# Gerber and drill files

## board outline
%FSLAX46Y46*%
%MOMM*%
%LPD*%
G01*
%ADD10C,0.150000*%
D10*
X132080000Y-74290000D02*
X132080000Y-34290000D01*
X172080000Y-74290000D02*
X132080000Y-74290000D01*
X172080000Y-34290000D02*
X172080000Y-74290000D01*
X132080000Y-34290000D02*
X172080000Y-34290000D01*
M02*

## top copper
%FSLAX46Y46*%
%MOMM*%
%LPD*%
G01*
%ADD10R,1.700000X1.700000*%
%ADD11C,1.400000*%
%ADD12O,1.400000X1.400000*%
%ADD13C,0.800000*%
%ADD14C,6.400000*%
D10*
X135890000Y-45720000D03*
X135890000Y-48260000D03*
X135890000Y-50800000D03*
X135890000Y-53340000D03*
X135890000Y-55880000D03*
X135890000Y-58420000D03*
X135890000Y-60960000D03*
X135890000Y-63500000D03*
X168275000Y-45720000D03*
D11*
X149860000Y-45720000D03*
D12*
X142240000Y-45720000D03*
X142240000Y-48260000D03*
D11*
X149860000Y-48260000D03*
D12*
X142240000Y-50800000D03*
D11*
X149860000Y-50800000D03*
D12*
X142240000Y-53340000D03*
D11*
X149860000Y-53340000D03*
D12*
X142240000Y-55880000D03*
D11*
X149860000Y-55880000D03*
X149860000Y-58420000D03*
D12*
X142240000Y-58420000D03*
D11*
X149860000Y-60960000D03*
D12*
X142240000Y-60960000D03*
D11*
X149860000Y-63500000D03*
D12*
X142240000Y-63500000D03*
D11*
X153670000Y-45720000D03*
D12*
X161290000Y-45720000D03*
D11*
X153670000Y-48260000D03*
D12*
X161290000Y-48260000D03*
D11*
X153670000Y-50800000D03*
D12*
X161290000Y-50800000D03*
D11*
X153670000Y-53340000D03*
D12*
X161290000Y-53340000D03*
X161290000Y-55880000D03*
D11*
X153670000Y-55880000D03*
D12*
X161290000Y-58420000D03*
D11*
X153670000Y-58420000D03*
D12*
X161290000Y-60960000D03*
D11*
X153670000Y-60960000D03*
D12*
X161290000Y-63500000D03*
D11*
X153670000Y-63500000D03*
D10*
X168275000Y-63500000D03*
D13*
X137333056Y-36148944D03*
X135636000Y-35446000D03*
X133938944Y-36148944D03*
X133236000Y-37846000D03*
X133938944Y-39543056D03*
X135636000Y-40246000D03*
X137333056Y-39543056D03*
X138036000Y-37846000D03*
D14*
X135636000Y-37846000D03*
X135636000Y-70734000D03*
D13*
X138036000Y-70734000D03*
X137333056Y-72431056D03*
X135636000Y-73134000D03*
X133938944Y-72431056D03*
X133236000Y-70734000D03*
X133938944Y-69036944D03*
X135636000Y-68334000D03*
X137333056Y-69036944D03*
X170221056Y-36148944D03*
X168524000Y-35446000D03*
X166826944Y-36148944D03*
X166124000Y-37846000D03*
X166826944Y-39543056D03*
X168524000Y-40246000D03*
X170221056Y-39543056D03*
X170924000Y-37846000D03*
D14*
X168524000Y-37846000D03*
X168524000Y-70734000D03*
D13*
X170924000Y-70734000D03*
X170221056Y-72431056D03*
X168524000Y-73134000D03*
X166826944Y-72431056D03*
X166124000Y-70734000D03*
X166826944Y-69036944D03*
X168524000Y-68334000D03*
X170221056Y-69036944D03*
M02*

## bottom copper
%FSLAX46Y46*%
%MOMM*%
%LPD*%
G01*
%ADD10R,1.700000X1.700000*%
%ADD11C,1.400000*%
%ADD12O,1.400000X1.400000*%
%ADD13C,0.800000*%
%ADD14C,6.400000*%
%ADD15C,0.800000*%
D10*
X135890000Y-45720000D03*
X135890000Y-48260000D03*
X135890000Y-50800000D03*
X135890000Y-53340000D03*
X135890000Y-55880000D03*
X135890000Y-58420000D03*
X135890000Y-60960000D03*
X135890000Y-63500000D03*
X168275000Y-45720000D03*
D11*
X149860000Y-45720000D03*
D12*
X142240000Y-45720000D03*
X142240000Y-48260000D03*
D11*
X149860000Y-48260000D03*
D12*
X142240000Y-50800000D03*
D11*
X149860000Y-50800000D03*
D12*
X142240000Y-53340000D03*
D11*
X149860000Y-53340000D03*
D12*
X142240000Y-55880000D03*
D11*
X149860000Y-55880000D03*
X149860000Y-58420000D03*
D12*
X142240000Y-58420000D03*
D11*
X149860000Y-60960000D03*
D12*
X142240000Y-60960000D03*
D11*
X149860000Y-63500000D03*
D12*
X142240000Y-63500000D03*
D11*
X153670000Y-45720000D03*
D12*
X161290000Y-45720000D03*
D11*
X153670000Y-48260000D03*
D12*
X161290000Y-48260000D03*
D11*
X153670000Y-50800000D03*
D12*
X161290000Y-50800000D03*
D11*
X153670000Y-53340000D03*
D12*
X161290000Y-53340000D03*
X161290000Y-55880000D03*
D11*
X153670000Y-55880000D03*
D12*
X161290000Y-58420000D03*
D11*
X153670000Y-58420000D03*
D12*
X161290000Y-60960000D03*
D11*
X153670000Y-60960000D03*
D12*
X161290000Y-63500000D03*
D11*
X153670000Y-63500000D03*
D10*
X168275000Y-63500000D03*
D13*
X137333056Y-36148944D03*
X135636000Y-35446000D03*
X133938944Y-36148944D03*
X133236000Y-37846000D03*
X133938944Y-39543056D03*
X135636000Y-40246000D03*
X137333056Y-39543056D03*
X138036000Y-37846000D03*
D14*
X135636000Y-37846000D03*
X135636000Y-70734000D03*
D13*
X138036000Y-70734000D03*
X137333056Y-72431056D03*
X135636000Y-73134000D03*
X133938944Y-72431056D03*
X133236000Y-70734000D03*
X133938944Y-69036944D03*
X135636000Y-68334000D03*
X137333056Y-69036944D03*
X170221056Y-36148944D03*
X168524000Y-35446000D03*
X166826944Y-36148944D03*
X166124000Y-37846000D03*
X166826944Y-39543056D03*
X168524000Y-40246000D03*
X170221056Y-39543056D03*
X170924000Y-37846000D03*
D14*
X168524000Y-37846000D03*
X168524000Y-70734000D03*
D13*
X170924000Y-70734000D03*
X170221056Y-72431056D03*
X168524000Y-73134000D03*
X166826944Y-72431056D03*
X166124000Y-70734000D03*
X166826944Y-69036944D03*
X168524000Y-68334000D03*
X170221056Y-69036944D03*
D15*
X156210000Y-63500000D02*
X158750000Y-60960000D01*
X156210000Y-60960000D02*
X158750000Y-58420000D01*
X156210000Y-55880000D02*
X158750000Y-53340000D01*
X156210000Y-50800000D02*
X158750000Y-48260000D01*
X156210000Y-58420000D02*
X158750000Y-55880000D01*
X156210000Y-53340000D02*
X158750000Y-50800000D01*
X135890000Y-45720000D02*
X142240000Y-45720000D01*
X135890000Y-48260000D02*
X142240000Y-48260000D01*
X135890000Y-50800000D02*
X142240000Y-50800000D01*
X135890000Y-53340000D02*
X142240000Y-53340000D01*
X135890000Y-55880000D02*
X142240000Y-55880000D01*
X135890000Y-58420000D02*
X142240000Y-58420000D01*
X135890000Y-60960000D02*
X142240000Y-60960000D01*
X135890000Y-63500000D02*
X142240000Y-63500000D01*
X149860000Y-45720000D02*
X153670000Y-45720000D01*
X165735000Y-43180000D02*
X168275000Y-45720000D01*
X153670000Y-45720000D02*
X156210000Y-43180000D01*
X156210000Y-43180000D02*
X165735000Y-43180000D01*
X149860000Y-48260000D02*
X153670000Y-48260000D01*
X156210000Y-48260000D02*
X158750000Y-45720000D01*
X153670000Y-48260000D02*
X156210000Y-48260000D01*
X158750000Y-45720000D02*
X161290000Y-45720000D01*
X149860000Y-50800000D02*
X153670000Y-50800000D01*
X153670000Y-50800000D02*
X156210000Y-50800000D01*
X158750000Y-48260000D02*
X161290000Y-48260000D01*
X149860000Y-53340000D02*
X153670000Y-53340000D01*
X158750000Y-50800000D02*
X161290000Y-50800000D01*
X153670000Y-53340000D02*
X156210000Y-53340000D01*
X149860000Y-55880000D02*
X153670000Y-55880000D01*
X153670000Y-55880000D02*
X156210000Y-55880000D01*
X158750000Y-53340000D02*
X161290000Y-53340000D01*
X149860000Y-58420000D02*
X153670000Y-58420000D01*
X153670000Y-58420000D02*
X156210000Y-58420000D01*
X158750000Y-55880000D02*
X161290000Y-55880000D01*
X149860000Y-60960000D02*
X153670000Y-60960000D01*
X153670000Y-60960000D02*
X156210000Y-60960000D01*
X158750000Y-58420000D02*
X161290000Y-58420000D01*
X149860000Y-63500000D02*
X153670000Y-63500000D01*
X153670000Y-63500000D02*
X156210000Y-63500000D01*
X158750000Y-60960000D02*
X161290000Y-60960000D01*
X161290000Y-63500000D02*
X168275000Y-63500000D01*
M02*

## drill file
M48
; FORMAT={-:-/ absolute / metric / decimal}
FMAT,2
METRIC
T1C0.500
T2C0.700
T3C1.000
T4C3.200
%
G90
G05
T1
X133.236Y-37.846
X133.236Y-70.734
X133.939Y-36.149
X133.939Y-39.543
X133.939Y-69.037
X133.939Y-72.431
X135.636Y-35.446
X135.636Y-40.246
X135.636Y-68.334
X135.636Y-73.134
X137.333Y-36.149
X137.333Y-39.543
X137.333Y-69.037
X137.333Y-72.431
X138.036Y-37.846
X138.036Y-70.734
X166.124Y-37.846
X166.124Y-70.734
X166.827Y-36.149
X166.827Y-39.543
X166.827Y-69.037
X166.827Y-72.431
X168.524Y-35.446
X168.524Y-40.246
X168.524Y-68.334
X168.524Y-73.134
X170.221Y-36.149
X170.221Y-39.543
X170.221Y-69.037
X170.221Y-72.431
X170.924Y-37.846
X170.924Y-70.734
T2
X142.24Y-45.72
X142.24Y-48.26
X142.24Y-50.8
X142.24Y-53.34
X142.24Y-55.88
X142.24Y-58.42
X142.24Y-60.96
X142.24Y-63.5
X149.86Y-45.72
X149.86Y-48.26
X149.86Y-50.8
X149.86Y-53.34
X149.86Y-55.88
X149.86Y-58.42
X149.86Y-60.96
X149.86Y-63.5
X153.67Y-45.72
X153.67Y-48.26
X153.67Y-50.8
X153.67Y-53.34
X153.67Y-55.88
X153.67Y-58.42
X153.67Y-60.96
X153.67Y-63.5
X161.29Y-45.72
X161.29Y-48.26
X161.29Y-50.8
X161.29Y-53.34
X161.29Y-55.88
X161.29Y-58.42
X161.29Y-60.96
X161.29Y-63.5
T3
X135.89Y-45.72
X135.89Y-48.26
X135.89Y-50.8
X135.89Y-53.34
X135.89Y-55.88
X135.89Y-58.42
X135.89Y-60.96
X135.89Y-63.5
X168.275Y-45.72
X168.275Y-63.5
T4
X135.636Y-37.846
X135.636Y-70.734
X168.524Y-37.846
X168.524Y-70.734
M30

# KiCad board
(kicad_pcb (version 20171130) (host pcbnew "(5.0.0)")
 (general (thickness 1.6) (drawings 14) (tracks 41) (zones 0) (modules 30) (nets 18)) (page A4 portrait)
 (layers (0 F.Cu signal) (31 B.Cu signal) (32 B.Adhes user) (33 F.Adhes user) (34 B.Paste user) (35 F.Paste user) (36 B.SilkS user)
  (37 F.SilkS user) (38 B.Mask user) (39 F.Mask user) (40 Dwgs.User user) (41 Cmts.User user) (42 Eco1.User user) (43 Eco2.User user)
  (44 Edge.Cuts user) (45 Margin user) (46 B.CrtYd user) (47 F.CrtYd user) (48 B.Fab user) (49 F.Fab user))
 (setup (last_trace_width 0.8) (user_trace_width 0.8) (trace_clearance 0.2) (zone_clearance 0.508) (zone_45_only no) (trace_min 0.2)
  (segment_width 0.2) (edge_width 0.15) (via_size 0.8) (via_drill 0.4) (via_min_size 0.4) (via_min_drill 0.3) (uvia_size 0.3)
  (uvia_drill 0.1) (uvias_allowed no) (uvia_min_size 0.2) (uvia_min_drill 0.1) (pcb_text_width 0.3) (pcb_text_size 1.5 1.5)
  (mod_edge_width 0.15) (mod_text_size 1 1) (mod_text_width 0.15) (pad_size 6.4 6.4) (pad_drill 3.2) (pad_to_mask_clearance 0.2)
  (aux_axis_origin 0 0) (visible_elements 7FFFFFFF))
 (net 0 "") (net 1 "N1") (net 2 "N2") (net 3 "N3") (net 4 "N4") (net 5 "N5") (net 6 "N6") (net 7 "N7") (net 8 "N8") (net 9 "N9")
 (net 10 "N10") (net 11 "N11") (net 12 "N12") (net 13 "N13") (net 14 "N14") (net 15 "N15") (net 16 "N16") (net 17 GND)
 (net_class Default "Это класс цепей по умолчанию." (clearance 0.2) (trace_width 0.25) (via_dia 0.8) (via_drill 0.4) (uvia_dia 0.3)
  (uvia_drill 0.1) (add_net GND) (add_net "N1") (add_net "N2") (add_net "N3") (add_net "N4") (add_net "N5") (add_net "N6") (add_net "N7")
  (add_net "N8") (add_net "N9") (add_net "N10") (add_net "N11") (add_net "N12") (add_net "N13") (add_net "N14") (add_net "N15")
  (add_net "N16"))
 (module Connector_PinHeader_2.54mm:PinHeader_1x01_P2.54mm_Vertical (layer F.Cu) (at 135.89 45.72)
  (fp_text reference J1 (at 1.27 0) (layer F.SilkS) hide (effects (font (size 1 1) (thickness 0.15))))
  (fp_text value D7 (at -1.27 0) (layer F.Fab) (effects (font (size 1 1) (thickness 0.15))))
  (pad 1 thru_hole rect (at 0 0) (size 1.7 1.7) (drill 1) (layers *.Cu *.Mask) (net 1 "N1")))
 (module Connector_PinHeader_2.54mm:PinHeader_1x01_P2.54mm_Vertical (layer F.Cu) (at 135.89 48.26)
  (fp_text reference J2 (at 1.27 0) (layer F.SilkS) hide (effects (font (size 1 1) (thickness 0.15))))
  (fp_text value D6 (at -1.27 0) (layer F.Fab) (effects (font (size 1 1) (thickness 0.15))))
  (pad 1 thru_hole rect (at 0 0) (size 1.7 1.7) (drill 1) (layers *.Cu *.Mask) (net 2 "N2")))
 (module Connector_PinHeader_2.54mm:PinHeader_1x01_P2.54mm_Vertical (layer F.Cu) (at 135.89 50.8)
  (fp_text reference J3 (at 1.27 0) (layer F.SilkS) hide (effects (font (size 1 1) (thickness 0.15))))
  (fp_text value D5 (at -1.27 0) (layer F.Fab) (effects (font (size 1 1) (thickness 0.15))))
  (pad 1 thru_hole rect (at 0 0) (size 1.7 1.7) (drill 1) (layers *.Cu *.Mask) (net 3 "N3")))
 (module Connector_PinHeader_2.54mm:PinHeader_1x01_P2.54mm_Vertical (layer F.Cu) (at 135.89 53.34)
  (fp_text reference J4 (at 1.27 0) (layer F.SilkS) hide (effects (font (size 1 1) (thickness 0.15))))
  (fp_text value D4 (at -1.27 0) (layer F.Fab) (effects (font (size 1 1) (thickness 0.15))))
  (pad 1 thru_hole rect (at 0 0) (size 1.7 1.7) (drill 1) (layers *.Cu *.Mask) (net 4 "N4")))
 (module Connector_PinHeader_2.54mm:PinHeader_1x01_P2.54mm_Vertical (layer F.Cu) (at 135.89 55.88)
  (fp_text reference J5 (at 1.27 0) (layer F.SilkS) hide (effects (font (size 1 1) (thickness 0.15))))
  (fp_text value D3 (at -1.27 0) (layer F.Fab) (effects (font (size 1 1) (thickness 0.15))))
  (pad 1 thru_hole rect (at 0 0) (size 1.7 1.7) (drill 1) (layers *.Cu *.Mask) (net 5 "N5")))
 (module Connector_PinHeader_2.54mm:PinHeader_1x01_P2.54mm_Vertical (layer F.Cu) (at 135.89 58.42)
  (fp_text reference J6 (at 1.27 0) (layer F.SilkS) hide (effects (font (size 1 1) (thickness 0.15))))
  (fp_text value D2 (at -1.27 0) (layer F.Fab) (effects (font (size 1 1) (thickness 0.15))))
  (pad 1 thru_hole rect (at 0 0) (size 1.7 1.7) (drill 1) (layers *.Cu *.Mask) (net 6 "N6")))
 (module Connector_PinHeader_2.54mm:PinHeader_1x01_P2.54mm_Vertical (layer F.Cu) (at 135.89 60.96)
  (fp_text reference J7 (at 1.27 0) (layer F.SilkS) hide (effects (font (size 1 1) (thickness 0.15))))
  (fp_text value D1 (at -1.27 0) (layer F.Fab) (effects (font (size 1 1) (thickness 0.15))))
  (pad 1 thru_hole rect (at 0 0) (size 1.7 1.7) (drill 1) (layers *.Cu *.Mask) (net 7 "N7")))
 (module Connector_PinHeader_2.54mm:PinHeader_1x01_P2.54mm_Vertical (layer F.Cu) (at 135.89 63.5)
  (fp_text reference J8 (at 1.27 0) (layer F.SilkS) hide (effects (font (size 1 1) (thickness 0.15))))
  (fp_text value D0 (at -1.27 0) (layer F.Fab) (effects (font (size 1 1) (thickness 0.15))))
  (pad 1 thru_hole rect (at 0 0) (size 1.7 1.7) (drill 1) (layers *.Cu *.Mask) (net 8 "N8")))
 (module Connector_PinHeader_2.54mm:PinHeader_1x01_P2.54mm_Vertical (layer F.Cu) (at 168.275 45.72)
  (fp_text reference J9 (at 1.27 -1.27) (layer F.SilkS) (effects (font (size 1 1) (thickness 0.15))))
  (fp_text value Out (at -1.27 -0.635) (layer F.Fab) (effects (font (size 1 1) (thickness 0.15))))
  (pad 1 thru_hole rect (at 0 0) (size 1.7 1.7) (drill 1) (layers *.Cu *.Mask) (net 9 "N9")))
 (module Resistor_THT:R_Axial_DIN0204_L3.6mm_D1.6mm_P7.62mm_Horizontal (layer F.Cu) (at 149.86 45.72 180)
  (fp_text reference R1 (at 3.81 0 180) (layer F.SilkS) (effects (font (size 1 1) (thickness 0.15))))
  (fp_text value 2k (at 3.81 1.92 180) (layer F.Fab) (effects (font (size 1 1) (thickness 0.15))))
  (pad 1 thru_hole circle (at 0 0 180) (size 1.4 1.4) (drill 0.7) (layers *.Cu *.Mask) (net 9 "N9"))
  (pad 2 thru_hole oval (at 7.62 0 180) (size 1.4 1.4) (drill 0.7) (layers *.Cu *.Mask) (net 1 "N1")))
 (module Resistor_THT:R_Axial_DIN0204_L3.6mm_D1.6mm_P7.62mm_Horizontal (layer F.Cu) (at 149.86 48.26 180)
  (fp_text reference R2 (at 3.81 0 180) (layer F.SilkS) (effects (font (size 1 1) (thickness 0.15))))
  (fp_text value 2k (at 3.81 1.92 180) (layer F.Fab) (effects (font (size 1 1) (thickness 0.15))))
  (pad 2 thru_hole oval (at 7.62 0 180) (size 1.4 1.4) (drill 0.7) (layers *.Cu *.Mask) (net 2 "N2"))
  (pad 1 thru_hole circle (at 0 0 180) (size 1.4 1.4) (drill 0.7) (layers *.Cu *.Mask) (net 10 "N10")))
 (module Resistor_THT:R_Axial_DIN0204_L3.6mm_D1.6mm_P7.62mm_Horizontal (layer F.Cu) (at 149.86 50.8 180)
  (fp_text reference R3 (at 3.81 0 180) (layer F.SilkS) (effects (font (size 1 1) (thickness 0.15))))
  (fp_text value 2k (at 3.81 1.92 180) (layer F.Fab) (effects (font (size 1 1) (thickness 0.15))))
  (pad 2 thru_hole oval (at 7.62 0 180) (size 1.4 1.4) (drill 0.7) (layers *.Cu *.Mask) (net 3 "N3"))
  (pad 1 thru_hole circle (at 0 0 180) (size 1.4 1.4) (drill 0.7) (layers *.Cu *.Mask) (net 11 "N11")))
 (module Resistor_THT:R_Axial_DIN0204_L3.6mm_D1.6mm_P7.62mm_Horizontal (layer F.Cu) (at 149.86 53.34 180)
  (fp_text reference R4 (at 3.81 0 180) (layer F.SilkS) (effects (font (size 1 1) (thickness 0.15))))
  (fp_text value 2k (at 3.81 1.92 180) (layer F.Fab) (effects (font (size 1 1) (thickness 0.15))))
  (pad 2 thru_hole oval (at 7.62 0 180) (size 1.4 1.4) (drill 0.7) (layers *.Cu *.Mask) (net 4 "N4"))
  (pad 1 thru_hole circle (at 0 0 180) (size 1.4 1.4) (drill 0.7) (layers *.Cu *.Mask) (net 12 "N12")))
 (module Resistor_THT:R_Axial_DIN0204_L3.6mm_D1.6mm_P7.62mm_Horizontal (layer F.Cu) (at 149.86 55.88 180)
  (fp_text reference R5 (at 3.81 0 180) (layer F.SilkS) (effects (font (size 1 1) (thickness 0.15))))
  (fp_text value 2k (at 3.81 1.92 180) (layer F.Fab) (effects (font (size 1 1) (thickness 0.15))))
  (pad 2 thru_hole oval (at 7.62 0 180) (size 1.4 1.4) (drill 0.7) (layers *.Cu *.Mask) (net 5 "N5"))
  (pad 1 thru_hole circle (at 0 0 180) (size 1.4 1.4) (drill 0.7) (layers *.Cu *.Mask) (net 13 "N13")))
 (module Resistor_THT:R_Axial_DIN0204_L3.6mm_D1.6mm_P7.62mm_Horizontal (layer F.Cu) (at 149.86 58.42 180)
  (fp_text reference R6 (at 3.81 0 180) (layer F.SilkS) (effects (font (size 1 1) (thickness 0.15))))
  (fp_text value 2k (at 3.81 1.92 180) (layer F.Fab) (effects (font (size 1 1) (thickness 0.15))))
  (pad 1 thru_hole circle (at 0 0 180) (size 1.4 1.4) (drill 0.7) (layers *.Cu *.Mask) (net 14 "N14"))
  (pad 2 thru_hole oval (at 7.62 0 180) (size 1.4 1.4) (drill 0.7) (layers *.Cu *.Mask) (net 6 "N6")))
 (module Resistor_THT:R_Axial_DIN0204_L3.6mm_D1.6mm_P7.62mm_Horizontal (layer F.Cu) (at 149.86 60.96 180)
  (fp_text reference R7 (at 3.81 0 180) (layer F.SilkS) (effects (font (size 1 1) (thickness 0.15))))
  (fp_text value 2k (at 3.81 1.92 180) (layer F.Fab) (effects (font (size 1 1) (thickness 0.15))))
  (pad 1 thru_hole circle (at 0 0 180) (size 1.4 1.4) (drill 0.7) (layers *.Cu *.Mask) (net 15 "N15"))
  (pad 2 thru_hole oval (at 7.62 0 180) (size 1.4 1.4) (drill 0.7) (layers *.Cu *.Mask) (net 7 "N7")))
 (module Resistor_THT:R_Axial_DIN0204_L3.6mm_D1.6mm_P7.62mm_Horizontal (layer F.Cu) (at 149.86 63.5 180)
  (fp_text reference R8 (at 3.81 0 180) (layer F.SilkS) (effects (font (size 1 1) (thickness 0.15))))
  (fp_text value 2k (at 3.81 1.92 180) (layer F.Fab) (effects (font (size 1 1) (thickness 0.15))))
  (pad 1 thru_hole circle (at 0 0 180) (size 1.4 1.4) (drill 0.7) (layers *.Cu *.Mask) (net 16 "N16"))
  (pad 2 thru_hole oval (at 7.62 0 180) (size 1.4 1.4) (drill 0.7) (layers *.Cu *.Mask) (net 8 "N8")))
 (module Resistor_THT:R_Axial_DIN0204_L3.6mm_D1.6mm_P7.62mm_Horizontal (layer F.Cu) (at 153.67 45.72)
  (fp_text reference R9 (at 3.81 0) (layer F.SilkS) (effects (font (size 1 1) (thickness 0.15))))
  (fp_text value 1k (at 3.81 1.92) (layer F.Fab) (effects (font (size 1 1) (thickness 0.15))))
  (pad 1 thru_hole circle (at 0 0) (size 1.4 1.4) (drill 0.7) (layers *.Cu *.Mask) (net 9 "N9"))
  (pad 2 thru_hole oval (at 7.62 0) (size 1.4 1.4) (drill 0.7) (layers *.Cu *.Mask) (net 10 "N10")))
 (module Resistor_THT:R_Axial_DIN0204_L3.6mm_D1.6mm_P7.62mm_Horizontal (layer F.Cu) (at 153.67 48.26)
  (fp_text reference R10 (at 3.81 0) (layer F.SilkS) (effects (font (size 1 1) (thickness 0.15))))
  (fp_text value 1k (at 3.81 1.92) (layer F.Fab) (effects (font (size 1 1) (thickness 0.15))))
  (pad 1 thru_hole circle (at 0 0) (size 1.4 1.4) (drill 0.7) (layers *.Cu *.Mask) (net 10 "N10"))
  (pad 2 thru_hole oval (at 7.62 0) (size 1.4 1.4) (drill 0.7) (layers *.Cu *.Mask) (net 11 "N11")))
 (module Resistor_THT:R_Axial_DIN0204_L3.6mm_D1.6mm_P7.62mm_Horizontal (layer F.Cu) (at 153.67 50.8)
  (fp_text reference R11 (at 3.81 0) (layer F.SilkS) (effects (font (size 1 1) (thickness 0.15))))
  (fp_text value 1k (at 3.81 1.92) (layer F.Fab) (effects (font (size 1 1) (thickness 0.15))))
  (pad 1 thru_hole circle (at 0 0) (size 1.4 1.4) (drill 0.7) (layers *.Cu *.Mask) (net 11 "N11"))
  (pad 2 thru_hole oval (at 7.62 0) (size 1.4 1.4) (drill 0.7) (layers *.Cu *.Mask) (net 12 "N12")))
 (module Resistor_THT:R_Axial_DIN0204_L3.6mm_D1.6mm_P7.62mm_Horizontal (layer F.Cu) (at 153.67 53.34)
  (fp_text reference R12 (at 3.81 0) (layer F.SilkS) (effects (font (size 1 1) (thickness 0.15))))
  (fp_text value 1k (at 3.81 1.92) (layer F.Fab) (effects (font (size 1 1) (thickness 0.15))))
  (pad 1 thru_hole circle (at 0 0) (size 1.4 1.4) (drill 0.7) (layers *.Cu *.Mask) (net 12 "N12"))
  (pad 2 thru_hole oval (at 7.62 0) (size 1.4 1.4) (drill 0.7) (layers *.Cu *.Mask) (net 13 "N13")))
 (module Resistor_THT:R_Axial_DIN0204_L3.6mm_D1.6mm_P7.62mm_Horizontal (layer F.Cu) (at 153.67 55.88)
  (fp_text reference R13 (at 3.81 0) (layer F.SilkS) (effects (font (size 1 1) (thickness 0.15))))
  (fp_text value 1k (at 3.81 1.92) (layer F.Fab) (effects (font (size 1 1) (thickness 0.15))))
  (pad 2 thru_hole oval (at 7.62 0) (size 1.4 1.4) (drill 0.7) (layers *.Cu *.Mask) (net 14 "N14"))
  (pad 1 thru_hole circle (at 0 0) (size 1.4 1.4) (drill 0.7) (layers *.Cu *.Mask) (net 13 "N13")))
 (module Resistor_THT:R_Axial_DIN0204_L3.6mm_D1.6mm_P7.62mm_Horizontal (layer F.Cu) (at 153.67 58.42)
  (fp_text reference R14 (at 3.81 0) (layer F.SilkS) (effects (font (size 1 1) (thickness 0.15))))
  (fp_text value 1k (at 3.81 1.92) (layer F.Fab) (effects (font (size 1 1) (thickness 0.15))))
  (pad 2 thru_hole oval (at 7.62 0) (size 1.4 1.4) (drill 0.7) (layers *.Cu *.Mask) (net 15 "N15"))
  (pad 1 thru_hole circle (at 0 0) (size 1.4 1.4) (drill 0.7) (layers *.Cu *.Mask) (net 14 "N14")))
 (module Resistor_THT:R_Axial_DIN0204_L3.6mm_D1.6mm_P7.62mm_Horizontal (layer F.Cu) (at 153.67 60.96)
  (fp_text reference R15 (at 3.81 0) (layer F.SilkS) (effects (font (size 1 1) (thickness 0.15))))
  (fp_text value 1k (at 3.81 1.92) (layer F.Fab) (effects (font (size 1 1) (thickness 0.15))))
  (pad 2 thru_hole oval (at 7.62 0) (size 1.4 1.4) (drill 0.7) (layers *.Cu *.Mask) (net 16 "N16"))
  (pad 1 thru_hole circle (at 0 0) (size 1.4 1.4) (drill 0.7) (layers *.Cu *.Mask) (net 15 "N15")))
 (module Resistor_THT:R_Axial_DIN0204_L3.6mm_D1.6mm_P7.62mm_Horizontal (layer F.Cu) (at 153.67 63.5)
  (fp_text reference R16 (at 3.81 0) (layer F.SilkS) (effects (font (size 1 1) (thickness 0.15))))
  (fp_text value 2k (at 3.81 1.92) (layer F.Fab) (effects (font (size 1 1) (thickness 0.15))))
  (pad 2 thru_hole oval (at 7.62 0) (size 1.4 1.4) (drill 0.7) (layers *.Cu *.Mask) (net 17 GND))
  (pad 1 thru_hole circle (at 0 0) (size 1.4 1.4) (drill 0.7) (layers *.Cu *.Mask) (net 16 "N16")))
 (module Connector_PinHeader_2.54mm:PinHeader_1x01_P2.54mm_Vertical (layer F.Cu) (at 168.275 63.5)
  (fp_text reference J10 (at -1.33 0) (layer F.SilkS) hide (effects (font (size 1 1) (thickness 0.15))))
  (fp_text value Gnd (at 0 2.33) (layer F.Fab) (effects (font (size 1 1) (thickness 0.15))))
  (pad 1 thru_hole rect (at 0 0) (size 1.7 1.7) (drill 1) (layers *.Cu *.Mask) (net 17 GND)))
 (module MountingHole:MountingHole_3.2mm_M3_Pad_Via (layer F.Cu) (at 135.636 37.846)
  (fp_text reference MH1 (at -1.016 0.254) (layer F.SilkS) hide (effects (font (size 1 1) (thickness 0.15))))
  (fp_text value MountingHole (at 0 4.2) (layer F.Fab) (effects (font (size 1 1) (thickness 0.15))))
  (pad 1 thru_hole circle (at 1.697056 -1.697056) (size 0.8 0.8) (drill 0.5) (layers *.Cu *.Mask))
  (pad 1 thru_hole circle (at 0 -2.4) (size 0.8 0.8) (drill 0.5) (layers *.Cu *.Mask))
  (pad 1 thru_hole circle (at -1.697056 -1.697056) (size 0.8 0.8) (drill 0.5) (layers *.Cu *.Mask))
  (pad 1 thru_hole circle (at -2.4 0) (size 0.8 0.8) (drill 0.5) (layers *.Cu *.Mask))
  (pad 1 thru_hole circle (at -1.697056 1.697056) (size 0.8 0.8) (drill 0.5) (layers *.Cu *.Mask))
  (pad 1 thru_hole circle (at 0 2.4) (size 0.8 0.8) (drill 0.5) (layers *.Cu *.Mask))
  (pad 1 thru_hole circle (at 1.697056 1.697056) (size 0.8 0.8) (drill 0.5) (layers *.Cu *.Mask))
  (pad 1 thru_hole circle (at 2.4 0) (size 0.8 0.8) (drill 0.5) (layers *.Cu *.Mask))
  (pad 1 thru_hole circle (at 0 0) (size 6.4 6.4) (drill 3.2) (layers *.Cu *.Mask)))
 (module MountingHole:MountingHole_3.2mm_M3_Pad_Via (layer F.Cu) (at 135.636 70.734)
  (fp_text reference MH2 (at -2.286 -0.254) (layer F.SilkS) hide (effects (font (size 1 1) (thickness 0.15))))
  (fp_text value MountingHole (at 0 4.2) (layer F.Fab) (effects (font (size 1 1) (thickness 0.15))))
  (pad 1 thru_hole circle (at 0 0) (size 6.4 6.4) (drill 3.2) (layers *.Cu *.Mask))
  (pad 1 thru_hole circle (at 2.4 0) (size 0.8 0.8) (drill 0.5) (layers *.Cu *.Mask))
  (pad 1 thru_hole circle (at 1.697056 1.697056) (size 0.8 0.8) (drill 0.5) (layers *.Cu *.Mask))
  (pad 1 thru_hole circle (at 0 2.4) (size 0.8 0.8) (drill 0.5) (layers *.Cu *.Mask))
  (pad 1 thru_hole circle (at -1.697056 1.697056) (size 0.8 0.8) (drill 0.5) (layers *.Cu *.Mask))
  (pad 1 thru_hole circle (at -2.4 0) (size 0.8 0.8) (drill 0.5) (layers *.Cu *.Mask))
  (pad 1 thru_hole circle (at -1.697056 -1.697056) (size 0.8 0.8) (drill 0.5) (layers *.Cu *.Mask))
  (pad 1 thru_hole circle (at 0 -2.4) (size 0.8 0.8) (drill 0.5) (layers *.Cu *.Mask))
  (pad 1 thru_hole circle (at 1.697056 -1.697056) (size 0.8 0.8) (drill 0.5) (layers *.Cu *.Mask)))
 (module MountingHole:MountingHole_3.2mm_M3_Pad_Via (layer F.Cu) (at 168.524 37.846)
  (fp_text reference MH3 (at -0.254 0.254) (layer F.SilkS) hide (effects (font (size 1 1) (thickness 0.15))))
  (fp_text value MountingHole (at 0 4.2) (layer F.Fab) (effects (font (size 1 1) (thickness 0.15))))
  (pad 1 thru_hole circle (at 1.697056 -1.697056) (size 0.8 0.8) (drill 0.5) (layers *.Cu *.Mask))
  (pad 1 thru_hole circle (at 0 -2.4) (size 0.8 0.8) (drill 0.5) (layers *.Cu *.Mask))
  (pad 1 thru_hole circle (at -1.697056 -1.697056) (size 0.8 0.8) (drill 0.5) (layers *.Cu *.Mask))
  (pad 1 thru_hole circle (at -2.4 0) (size 0.8 0.8) (drill 0.5) (layers *.Cu *.Mask))
  (pad 1 thru_hole circle (at -1.697056 1.697056) (size 0.8 0.8) (drill 0.5) (layers *.Cu *.Mask))
  (pad 1 thru_hole circle (at 0 2.4) (size 0.8 0.8) (drill 0.5) (layers *.Cu *.Mask))
  (pad 1 thru_hole circle (at 1.697056 1.697056) (size 0.8 0.8) (drill 0.5) (layers *.Cu *.Mask))
  (pad 1 thru_hole circle (at 2.4 0) (size 0.8 0.8) (drill 0.5) (layers *.Cu *.Mask))
  (pad 1 thru_hole circle (at 0 0) (size 6.4 6.4) (drill 3.2) (layers *.Cu *.Mask)))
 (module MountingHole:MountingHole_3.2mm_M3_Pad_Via (layer F.Cu) (at 168.524 70.734)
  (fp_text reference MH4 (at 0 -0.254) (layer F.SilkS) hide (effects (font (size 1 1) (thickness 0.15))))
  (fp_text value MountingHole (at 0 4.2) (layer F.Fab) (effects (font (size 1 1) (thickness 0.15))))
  (pad 1 thru_hole circle (at 0 0) (size 6.4 6.4) (drill 3.2) (layers *.Cu *.Mask))
  (pad 1 thru_hole circle (at 2.4 0) (size 0.8 0.8) (drill 0.5) (layers *.Cu *.Mask))
  (pad 1 thru_hole circle (at 1.697056 1.697056) (size 0.8 0.8) (drill 0.5) (layers *.Cu *.Mask))
  (pad 1 thru_hole circle (at 0 2.4) (size 0.8 0.8) (drill 0.5) (layers *.Cu *.Mask))
  (pad 1 thru_hole circle (at -1.697056 1.697056) (size 0.8 0.8) (drill 0.5) (layers *.Cu *.Mask))
  (pad 1 thru_hole circle (at -2.4 0) (size 0.8 0.8) (drill 0.5) (layers *.Cu *.Mask))
  (pad 1 thru_hole circle (at -1.697056 -1.697056) (size 0.8 0.8) (drill 0.5) (layers *.Cu *.Mask))
  (pad 1 thru_hole circle (at 0 -2.4) (size 0.8 0.8) (drill 0.5) (layers *.Cu *.Mask))
  (pad 1 thru_hole circle (at 1.697056 -1.697056) (size 0.8 0.8) (drill 0.5) (layers *.Cu *.Mask)))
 (gr_line (start 132.08 74.29) (end 132.08 34.29) (layer Edge.Cuts) (width 0.15))
 (gr_line (start 172.08 74.29) (end 132.08 74.29) (layer Edge.Cuts) (width 0.15))
 (gr_line (start 172.08 34.29) (end 172.08 74.29) (layer Edge.Cuts) (width 0.15))
 (gr_line (start 132.08 34.29) (end 172.08 34.29) (layer Edge.Cuts) (width 0.15))
 (segment (start 156.21 63.5) (end 158.75 60.96) (width 0.8) (layer B.Cu) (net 16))
 (segment (start 156.21 60.96) (end 158.75 58.42) (width 0.8) (layer B.Cu) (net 15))
 (segment (start 156.21 55.88) (end 158.75 53.34) (width 0.8) (layer B.Cu) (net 13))
 (segment (start 156.21 50.8) (end 158.75 48.26) (width 0.8) (layer B.Cu) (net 11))
 (segment (start 156.21 58.42) (end 158.75 55.88) (width 0.8) (layer B.Cu) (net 14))
 (segment (start 156.21 53.34) (end 158.75 50.8) (width 0.8) (layer B.Cu) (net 12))
 (segment (start 135.89 45.72) (end 142.24 45.72) (width 0.8) (layer B.Cu) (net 1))
 (segment (start 135.89 48.26) (end 142.24 48.26) (width 0.8) (layer B.Cu) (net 2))
 (segment (start 135.89 50.8) (end 142.24 50.8) (width 0.8) (layer B.Cu) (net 3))
 (segment (start 135.89 53.34) (end 142.24 53.34) (width 0.8) (layer B.Cu) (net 4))
 (segment (start 135.89 55.88) (end 142.24 55.88) (width 0.8) (layer B.Cu) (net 5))
 (segment (start 135.89 58.42) (end 142.24 58.42) (width 0.8) (layer B.Cu) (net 6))
 (segment (start 135.89 60.96) (end 142.24 60.96) (width 0.8) (layer B.Cu) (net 7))
 (segment (start 135.89 63.5) (end 142.24 63.5) (width 0.8) (layer B.Cu) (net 8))
 (segment (start 149.86 45.72) (end 153.67 45.72) (width 0.8) (layer B.Cu) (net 9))
 (segment (start 165.735 43.18) (end 168.275 45.72) (width 0.8) (layer B.Cu) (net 9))
 (segment (start 153.67 45.72) (end 156.21 43.18) (width 0.8) (layer B.Cu) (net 9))
 (segment (start 156.21 43.18) (end 165.735 43.18) (width 0.8) (layer B.Cu) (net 9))
 (segment (start 149.86 48.26) (end 153.67 48.26) (width 0.8) (layer B.Cu) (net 10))
 (segment (start 156.21 48.26) (end 158.75 45.72) (width 0.8) (layer B.Cu) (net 10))
 (segment (start 153.67 48.26) (end 156.21 48.26) (width 0.8) (layer B.Cu) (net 10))
 (segment (start 158.75 45.72) (end 161.29 45.72) (width 0.8) (layer B.Cu) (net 10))
 (segment (start 149.86 50.8) (end 153.67 50.8) (width 0.8) (layer B.Cu) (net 11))
 (segment (start 153.67 50.8) (end 156.21 50.8) (width 0.8) (layer B.Cu) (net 11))
 (segment (start 158.75 48.26) (end 161.29 48.26) (width 0.8) (layer B.Cu) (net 11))
 (segment (start 149.86 53.34) (end 153.67 53.34) (width 0.8) (layer B.Cu) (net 12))
 (segment (start 158.75 50.8) (end 161.29 50.8) (width 0.8) (layer B.Cu) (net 12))
 (segment (start 153.67 53.34) (end 156.21 53.34) (width 0.8) (layer B.Cu) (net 12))
 (segment (start 149.86 55.88) (end 153.67 55.88) (width 0.8) (layer B.Cu) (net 13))
 (segment (start 153.67 55.88) (end 156.21 55.88) (width 0.8) (layer B.Cu) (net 13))
 (segment (start 158.75 53.34) (end 161.29 53.34) (width 0.8) (layer B.Cu) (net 13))
 (segment (start 149.86 58.42) (end 153.67 58.42) (width 0.8) (layer B.Cu) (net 14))
 (segment (start 153.67 58.42) (end 156.21 58.42) (width 0.8) (layer B.Cu) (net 14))
 (segment (start 158.75 55.88) (end 161.29 55.88) (width 0.8) (layer B.Cu) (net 14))
 (segment (start 149.86 60.96) (end 153.67 60.96) (width 0.8) (layer B.Cu) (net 15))
 (segment (start 153.67 60.96) (end 156.21 60.96) (width 0.8) (layer B.Cu) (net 15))
 (segment (start 158.75 58.42) (end 161.29 58.42) (width 0.8) (layer B.Cu) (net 15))
 (segment (start 149.86 63.5) (end 153.67 63.5) (width 0.8) (layer B.Cu) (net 16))
 (segment (start 153.67 63.5) (end 156.21 63.5) (width 0.8) (layer B.Cu) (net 16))
 (segment (start 158.75 60.96) (end 161.29 60.96) (width 0.8) (layer B.Cu) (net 16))
 (segment (start 161.29 63.5) (end 168.275 63.5) (width 0.8) (layer B.Cu) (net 17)))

